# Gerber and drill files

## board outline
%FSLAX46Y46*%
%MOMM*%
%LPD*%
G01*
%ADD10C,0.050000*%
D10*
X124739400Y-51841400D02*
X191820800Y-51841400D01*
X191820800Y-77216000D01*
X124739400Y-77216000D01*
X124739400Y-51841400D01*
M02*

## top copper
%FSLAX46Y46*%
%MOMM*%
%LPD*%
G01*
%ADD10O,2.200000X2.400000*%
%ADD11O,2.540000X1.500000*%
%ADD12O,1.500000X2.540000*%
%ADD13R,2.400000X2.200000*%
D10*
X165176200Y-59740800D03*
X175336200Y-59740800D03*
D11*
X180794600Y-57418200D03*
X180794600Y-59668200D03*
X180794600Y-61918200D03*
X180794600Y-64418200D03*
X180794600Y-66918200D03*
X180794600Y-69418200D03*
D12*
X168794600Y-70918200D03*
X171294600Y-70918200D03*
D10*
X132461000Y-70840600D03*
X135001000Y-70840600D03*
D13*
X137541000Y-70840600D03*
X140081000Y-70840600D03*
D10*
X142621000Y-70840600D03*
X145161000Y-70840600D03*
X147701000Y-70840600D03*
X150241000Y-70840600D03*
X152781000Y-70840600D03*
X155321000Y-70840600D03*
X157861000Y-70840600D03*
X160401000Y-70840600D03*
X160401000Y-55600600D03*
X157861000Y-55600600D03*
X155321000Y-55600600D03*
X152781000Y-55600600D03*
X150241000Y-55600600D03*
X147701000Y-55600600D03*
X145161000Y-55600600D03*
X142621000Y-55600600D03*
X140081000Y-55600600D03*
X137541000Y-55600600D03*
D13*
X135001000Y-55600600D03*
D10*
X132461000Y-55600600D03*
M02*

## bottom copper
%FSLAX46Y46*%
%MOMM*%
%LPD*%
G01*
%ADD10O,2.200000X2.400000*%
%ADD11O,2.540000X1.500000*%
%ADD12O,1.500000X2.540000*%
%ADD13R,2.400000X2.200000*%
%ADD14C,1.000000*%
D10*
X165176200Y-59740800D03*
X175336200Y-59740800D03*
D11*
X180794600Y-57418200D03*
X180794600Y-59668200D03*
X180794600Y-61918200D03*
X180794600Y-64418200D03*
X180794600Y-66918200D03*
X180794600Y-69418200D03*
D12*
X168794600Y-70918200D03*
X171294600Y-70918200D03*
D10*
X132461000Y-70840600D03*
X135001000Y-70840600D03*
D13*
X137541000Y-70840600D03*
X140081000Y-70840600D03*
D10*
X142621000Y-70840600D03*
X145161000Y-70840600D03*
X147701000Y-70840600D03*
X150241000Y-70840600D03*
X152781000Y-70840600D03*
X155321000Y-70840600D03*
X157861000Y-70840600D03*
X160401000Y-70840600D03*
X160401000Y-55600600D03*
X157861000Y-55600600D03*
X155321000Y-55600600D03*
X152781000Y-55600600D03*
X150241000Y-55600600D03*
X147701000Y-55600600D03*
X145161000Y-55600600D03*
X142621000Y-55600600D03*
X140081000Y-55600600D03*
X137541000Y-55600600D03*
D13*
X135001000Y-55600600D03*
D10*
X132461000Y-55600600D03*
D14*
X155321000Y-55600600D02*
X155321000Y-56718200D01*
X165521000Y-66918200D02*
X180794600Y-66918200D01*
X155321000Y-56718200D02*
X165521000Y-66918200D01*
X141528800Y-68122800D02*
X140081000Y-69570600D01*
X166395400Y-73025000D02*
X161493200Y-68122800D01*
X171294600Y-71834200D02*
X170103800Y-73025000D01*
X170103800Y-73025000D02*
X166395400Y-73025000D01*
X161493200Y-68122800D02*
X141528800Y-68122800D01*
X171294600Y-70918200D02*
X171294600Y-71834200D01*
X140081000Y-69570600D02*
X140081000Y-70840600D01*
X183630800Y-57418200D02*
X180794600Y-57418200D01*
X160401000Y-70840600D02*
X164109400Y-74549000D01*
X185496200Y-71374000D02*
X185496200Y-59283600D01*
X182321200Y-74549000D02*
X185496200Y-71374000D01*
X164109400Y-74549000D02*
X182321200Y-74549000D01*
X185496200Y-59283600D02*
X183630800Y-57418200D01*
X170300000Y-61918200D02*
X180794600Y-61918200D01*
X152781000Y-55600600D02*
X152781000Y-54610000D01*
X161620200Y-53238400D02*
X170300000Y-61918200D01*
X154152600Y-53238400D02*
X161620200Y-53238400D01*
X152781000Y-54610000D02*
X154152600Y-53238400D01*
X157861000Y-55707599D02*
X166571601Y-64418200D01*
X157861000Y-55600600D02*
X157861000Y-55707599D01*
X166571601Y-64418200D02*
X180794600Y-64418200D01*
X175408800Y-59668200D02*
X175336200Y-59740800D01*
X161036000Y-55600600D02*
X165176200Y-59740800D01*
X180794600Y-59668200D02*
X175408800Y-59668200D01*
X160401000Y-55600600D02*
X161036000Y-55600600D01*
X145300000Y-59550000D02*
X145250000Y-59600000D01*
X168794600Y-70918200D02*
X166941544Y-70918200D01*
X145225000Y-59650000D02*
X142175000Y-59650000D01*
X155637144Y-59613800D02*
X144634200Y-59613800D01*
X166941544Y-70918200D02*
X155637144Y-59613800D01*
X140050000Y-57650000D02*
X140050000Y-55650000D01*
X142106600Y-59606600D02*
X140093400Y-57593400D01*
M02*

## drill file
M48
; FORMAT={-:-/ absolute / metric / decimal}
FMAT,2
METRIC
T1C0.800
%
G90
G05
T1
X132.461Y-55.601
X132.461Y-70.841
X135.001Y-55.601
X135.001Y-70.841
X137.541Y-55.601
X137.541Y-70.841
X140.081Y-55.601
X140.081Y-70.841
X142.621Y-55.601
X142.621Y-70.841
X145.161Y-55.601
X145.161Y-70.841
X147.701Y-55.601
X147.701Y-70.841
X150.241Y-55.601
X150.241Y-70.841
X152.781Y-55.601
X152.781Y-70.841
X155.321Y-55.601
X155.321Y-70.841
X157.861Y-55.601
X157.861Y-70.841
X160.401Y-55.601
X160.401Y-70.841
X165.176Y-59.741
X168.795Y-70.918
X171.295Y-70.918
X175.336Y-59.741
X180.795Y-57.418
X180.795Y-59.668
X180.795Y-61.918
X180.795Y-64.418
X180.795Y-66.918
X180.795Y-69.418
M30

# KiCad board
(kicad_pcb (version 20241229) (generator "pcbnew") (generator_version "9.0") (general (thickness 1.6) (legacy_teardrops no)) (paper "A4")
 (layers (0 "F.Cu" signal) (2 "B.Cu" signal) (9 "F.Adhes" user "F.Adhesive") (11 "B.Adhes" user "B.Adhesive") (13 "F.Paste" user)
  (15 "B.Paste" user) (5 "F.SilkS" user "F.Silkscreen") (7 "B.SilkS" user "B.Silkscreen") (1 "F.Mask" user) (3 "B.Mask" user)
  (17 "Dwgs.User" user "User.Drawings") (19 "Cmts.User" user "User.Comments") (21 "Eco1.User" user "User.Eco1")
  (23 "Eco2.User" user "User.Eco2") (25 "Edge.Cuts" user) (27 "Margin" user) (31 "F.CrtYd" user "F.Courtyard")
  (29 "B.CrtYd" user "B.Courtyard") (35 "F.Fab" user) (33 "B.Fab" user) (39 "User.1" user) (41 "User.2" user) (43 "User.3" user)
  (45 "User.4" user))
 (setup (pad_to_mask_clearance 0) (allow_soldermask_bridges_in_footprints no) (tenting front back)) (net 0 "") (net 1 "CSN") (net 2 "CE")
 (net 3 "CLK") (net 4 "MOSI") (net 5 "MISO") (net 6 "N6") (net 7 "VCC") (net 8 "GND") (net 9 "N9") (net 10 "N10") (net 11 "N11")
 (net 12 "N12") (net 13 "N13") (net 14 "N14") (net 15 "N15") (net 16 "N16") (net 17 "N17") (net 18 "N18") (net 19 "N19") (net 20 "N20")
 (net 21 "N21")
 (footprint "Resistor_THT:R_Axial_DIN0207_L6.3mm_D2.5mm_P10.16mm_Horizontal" (layer "F.Cu") (at 165.1762 59.7408)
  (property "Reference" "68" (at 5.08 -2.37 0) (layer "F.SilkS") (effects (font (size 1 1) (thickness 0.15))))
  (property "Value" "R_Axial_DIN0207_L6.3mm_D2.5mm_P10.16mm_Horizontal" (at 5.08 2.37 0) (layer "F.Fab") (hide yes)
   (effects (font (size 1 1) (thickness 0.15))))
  (pad "1" thru_hole oval (at 0 0 90) (size 2.4 2.2) (drill 0.8) (layers "*.Cu" "*.Mask") (remove_unused_layers no) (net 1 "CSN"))
  (pad "2" thru_hole oval (at 10.16 0 90) (size 2.4 2.2) (drill 0.8) (layers "*.Cu" "*.Mask") (remove_unused_layers no) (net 1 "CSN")))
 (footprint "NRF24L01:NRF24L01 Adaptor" (layer "F.Cu") (at 177.5446 63.4182)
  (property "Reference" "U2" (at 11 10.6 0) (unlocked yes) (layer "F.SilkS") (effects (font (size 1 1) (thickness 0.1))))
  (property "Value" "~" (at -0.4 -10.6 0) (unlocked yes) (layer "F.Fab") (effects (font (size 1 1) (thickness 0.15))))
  (pad "1" thru_hole oval (at 3.25 -6) (size 2.54 1.5) (drill 0.8) (layers "*.Cu" "*.Mask") (remove_unused_layers no) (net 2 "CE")
   (thermal_bridge_angle 45))
  (pad "2" thru_hole oval (at 3.25 -3.75) (size 2.54 1.5) (drill 0.8) (layers "*.Cu" "*.Mask") (remove_unused_layers no) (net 1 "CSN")
   (thermal_bridge_angle 45))
  (pad "3" thru_hole oval (at 3.25 -1.5) (size 2.54 1.5) (drill 0.8) (layers "*.Cu" "*.Mask") (remove_unused_layers no) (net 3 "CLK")
   (thermal_bridge_angle 45))
  (pad "4" thru_hole oval (at 3.25 1) (size 2.54 1.5) (drill 0.8) (layers "*.Cu" "*.Mask") (remove_unused_layers no) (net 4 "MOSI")
   (thermal_bridge_angle 45))
  (pad "5" thru_hole oval (at 3.25 3.5) (size 2.54 1.5) (drill 0.8) (layers "*.Cu" "*.Mask") (remove_unused_layers no) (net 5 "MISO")
   (thermal_bridge_angle 45))
  (pad "6" thru_hole oval (at 3.25 6) (size 2.54 1.5) (drill 0.8) (layers "*.Cu" "*.Mask") (remove_unused_layers no) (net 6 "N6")
   (thermal_bridge_angle 45))
  (pad "7" thru_hole oval (at -8.75 7.5) (size 1.5 2.54) (drill 0.8) (layers "*.Cu" "*.Mask") (remove_unused_layers no) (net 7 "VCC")
   (thermal_bridge_angle 45))
  (pad "8" thru_hole oval (at -6.25 7.5) (size 1.5 2.54) (drill 0.8) (layers "*.Cu" "*.Mask") (remove_unused_layers no) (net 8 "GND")
   (thermal_bridge_angle 45))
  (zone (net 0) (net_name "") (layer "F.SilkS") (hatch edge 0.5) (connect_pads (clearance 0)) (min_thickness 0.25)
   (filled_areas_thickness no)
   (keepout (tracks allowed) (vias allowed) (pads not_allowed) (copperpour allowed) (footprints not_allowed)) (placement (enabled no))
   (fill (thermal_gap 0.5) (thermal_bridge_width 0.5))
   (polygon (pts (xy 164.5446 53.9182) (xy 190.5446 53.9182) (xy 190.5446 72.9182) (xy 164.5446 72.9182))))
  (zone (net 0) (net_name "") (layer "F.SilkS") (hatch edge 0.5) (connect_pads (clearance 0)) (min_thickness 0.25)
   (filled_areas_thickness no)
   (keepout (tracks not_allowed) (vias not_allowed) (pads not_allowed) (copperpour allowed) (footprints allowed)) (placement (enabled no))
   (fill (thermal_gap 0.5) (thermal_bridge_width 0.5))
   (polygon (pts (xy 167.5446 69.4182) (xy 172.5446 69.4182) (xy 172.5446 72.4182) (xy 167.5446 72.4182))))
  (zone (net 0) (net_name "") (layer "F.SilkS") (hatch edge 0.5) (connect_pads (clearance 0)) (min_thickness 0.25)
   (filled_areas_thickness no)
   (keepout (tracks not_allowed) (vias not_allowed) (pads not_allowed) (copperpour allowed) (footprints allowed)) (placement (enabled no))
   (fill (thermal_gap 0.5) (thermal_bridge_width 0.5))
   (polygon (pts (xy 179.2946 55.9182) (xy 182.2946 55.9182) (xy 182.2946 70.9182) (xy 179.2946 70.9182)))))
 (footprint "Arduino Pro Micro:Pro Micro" (layer "F.Cu") (at 146.431 63.2206)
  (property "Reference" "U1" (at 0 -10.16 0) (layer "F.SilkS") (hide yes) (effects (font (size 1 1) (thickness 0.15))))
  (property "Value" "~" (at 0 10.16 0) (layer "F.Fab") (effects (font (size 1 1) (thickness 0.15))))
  (pad "1" thru_hole oval (at -13.97 7.62 90) (size 2.4 2.2) (drill 0.8) (layers "*.Cu" "*.Mask") (remove_unused_layers no) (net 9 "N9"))
  (pad "2" thru_hole oval (at -11.43 7.62 90) (size 2.4 2.2) (drill 0.8) (layers "*.Cu" "*.Mask") (remove_unused_layers no) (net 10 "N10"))
  (pad "3" thru_hole rect (at -8.89 7.62) (size 2.4 2.2) (drill 0.8) (layers "*.Cu" "*.Mask") (remove_unused_layers no) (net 8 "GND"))
  (pad "4" thru_hole rect (at -6.35 7.62) (size 2.4 2.2) (drill 0.8) (layers "*.Cu" "*.Mask") (remove_unused_layers no) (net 8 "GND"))
  (pad "5" thru_hole oval (at -3.81 7.62 90) (size 2.4 2.2) (drill 0.8) (layers "*.Cu" "*.Mask") (remove_unused_layers no) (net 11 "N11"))
  (pad "6" thru_hole oval (at -1.27 7.62 90) (size 2.4 2.2) (drill 0.8) (layers "*.Cu" "*.Mask") (remove_unused_layers no) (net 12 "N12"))
  (pad "7" thru_hole oval (at 1.27 7.62 90) (size 2.4 2.2) (drill 0.8) (layers "*.Cu" "*.Mask") (remove_unused_layers no) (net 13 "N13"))
  (pad "8" thru_hole oval (at 3.81 7.62 90) (size 2.4 2.2) (drill 0.8) (layers "*.Cu" "*.Mask") (remove_unused_layers no) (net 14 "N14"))
  (pad "9" thru_hole oval (at 6.35 7.62 90) (size 2.4 2.2) (drill 0.8) (layers "*.Cu" "*.Mask") (remove_unused_layers no) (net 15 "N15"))
  (pad "10" thru_hole oval (at 8.89 7.62 90) (size 2.4 2.2) (drill 0.8) (layers "*.Cu" "*.Mask") (remove_unused_layers no) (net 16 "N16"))
  (pad "11" thru_hole oval (at 11.43 7.62 90) (size 2.4 2.2) (drill 0.8) (layers "*.Cu" "*.Mask") (remove_unused_layers no))
  (pad "12" thru_hole oval (at 13.97 7.62 90) (size 2.4 2.2) (drill 0.8) (layers "*.Cu" "*.Mask") (remove_unused_layers no) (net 2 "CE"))
  (pad "13" thru_hole oval (at 13.97 -7.62 90) (size 2.4 2.2) (drill 0.8) (layers "*.Cu" "*.Mask") (remove_unused_layers no) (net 1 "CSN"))
  (pad "14" thru_hole oval (at 11.43 -7.62 90) (size 2.4 2.2) (drill 0.8) (layers "*.Cu" "*.Mask") (remove_unused_layers no) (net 4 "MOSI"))
  (pad "15" thru_hole oval (at 8.89 -7.62 90) (size 2.4 2.2) (drill 0.8) (layers "*.Cu" "*.Mask") (remove_unused_layers no) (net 5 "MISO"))
  (pad "16" thru_hole oval (at 6.35 -7.62 90) (size 2.4 2.2) (drill 0.8) (layers "*.Cu" "*.Mask") (remove_unused_layers no) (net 3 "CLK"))
  (pad "17" thru_hole oval (at 3.81 -7.62 90) (size 2.4 2.2) (drill 0.8) (layers "*.Cu" "*.Mask") (remove_unused_layers no) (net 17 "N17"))
  (pad "18" thru_hole oval (at 1.27 -7.62 90) (size 2.4 2.2) (drill 0.8) (layers "*.Cu" "*.Mask") (remove_unused_layers no) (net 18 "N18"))
  (pad "19" thru_hole oval (at -1.27 -7.62 90) (size 2.4 2.2) (drill 0.8) (layers "*.Cu" "*.Mask") (remove_unused_layers no) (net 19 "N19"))
  (pad "20" thru_hole oval (at -3.81 -7.62 90) (size 2.4 2.2) (drill 0.8) (layers "*.Cu" "*.Mask") (remove_unused_layers no) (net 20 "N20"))
  (pad "21" thru_hole oval (at -6.35 -7.62 90) (size 2.4 2.2) (drill 0.8) (layers "*.Cu" "*.Mask") (remove_unused_layers no) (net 7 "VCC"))
  (pad "22" thru_hole oval (at -8.89 -7.62 90) (size 2.4 2.2) (drill 0.8) (layers "*.Cu" "*.Mask") (remove_unused_layers no) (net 8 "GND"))
  (pad "23" thru_hole rect (at -11.43 -7.62) (size 2.4 2.2) (drill 0.8) (layers "*.Cu" "*.Mask") (remove_unused_layers no) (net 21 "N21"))
  (pad "24" thru_hole oval (at -13.97 -7.62 90) (size 2.4 2.2) (drill 0.8) (layers "*.Cu" "*.Mask") (remove_unused_layers no)))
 (gr_rect (start 124.7394 51.8414) (end 191.8208 77.216) (stroke (width 0.05) (type default)) (fill no) (layer "Edge.Cuts"))
 (segment (start 155.321 55.6006) (end 155.321 56.7182) (width 1) (layer "B.Cu") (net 5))
 (segment (start 165.521 66.9182) (end 180.7946 66.9182) (width 1) (layer "B.Cu") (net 5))
 (segment (start 155.321 56.7182) (end 165.521 66.9182) (width 1) (layer "B.Cu") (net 5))
 (segment (start 141.5288 68.1228) (end 140.081 69.5706) (width 1) (layer "B.Cu") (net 8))
 (segment (start 166.3954 73.025) (end 161.4932 68.1228) (width 1) (layer "B.Cu") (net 8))
 (segment (start 171.2946 71.8342) (end 170.1038 73.025) (width 1) (layer "B.Cu") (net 8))
 (segment (start 170.1038 73.025) (end 166.3954 73.025) (width 1) (layer "B.Cu") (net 8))
 (segment (start 161.4932 68.1228) (end 141.5288 68.1228) (width 1) (layer "B.Cu") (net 8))
 (segment (start 171.2946 70.9182) (end 171.2946 71.8342) (width 1) (layer "B.Cu") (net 8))
 (segment (start 140.081 69.5706) (end 140.081 70.8406) (width 1) (layer "B.Cu") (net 8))
 (segment (start 183.6308 57.4182) (end 180.7946 57.4182) (width 1) (layer "B.Cu") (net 2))
 (segment (start 160.401 70.8406) (end 164.1094 74.549) (width 1) (layer "B.Cu") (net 2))
 (segment (start 185.4962 71.374) (end 185.4962 59.2836) (width 1) (layer "B.Cu") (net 2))
 (segment (start 182.3212 74.549) (end 185.4962 71.374) (width 1) (layer "B.Cu") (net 2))
 (segment (start 164.1094 74.549) (end 182.3212 74.549) (width 1) (layer "B.Cu") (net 2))
 (segment (start 185.4962 59.2836) (end 183.6308 57.4182) (width 1) (layer "B.Cu") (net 2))
 (segment (start 170.3 61.9182) (end 180.7946 61.9182) (width 1) (layer "B.Cu") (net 3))
 (segment (start 152.781 55.6006) (end 152.781 54.61) (width 1) (layer "B.Cu") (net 3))
 (segment (start 161.6202 53.2384) (end 170.3 61.9182) (width 1) (layer "B.Cu") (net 3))
 (segment (start 154.1526 53.2384) (end 161.6202 53.2384) (width 1) (layer "B.Cu") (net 3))
 (segment (start 152.781 54.61) (end 154.1526 53.2384) (width 1) (layer "B.Cu") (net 3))
 (segment (start 157.861 55.707599) (end 166.571601 64.4182) (width 1) (layer "B.Cu") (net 4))
 (segment (start 157.861 55.6006) (end 157.861 55.707599) (width 1) (layer "B.Cu") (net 4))
 (segment (start 166.571601 64.4182) (end 180.7946 64.4182) (width 1) (layer "B.Cu") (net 4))
 (segment (start 175.4088 59.6682) (end 175.3362 59.7408) (width 1) (layer "B.Cu") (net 1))
 (segment (start 161.036 55.6006) (end 165.1762 59.7408) (width 1) (layer "B.Cu") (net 1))
 (segment (start 180.7946 59.6682) (end 175.4088 59.6682) (width 1) (layer "B.Cu") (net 1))
 (segment (start 160.401 55.6006) (end 161.036 55.6006) (width 1) (layer "B.Cu") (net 1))
 (segment (start 145.3 59.55) (end 145.25 59.6) (width 1) (layer "B.Cu") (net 7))
 (segment (start 168.7946 70.9182) (end 166.941544 70.9182) (width 1) (layer "B.Cu") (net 7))
 (segment (start 145.225 59.65) (end 142.175 59.65) (width 1) (layer "B.Cu") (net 7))
 (segment (start 155.637144 59.6138) (end 144.6342 59.6138) (width 1) (layer "B.Cu") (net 7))
 (segment (start 166.941544 70.9182) (end 155.637144 59.6138) (width 1) (layer "B.Cu") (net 7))
 (segment (start 140.05 57.65) (end 140.05 55.65) (width 1) (layer "B.Cu") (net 7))
 (segment (start 142.1066 59.6066) (end 140.0934 57.5934) (width 1) (layer "B.Cu") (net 7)))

